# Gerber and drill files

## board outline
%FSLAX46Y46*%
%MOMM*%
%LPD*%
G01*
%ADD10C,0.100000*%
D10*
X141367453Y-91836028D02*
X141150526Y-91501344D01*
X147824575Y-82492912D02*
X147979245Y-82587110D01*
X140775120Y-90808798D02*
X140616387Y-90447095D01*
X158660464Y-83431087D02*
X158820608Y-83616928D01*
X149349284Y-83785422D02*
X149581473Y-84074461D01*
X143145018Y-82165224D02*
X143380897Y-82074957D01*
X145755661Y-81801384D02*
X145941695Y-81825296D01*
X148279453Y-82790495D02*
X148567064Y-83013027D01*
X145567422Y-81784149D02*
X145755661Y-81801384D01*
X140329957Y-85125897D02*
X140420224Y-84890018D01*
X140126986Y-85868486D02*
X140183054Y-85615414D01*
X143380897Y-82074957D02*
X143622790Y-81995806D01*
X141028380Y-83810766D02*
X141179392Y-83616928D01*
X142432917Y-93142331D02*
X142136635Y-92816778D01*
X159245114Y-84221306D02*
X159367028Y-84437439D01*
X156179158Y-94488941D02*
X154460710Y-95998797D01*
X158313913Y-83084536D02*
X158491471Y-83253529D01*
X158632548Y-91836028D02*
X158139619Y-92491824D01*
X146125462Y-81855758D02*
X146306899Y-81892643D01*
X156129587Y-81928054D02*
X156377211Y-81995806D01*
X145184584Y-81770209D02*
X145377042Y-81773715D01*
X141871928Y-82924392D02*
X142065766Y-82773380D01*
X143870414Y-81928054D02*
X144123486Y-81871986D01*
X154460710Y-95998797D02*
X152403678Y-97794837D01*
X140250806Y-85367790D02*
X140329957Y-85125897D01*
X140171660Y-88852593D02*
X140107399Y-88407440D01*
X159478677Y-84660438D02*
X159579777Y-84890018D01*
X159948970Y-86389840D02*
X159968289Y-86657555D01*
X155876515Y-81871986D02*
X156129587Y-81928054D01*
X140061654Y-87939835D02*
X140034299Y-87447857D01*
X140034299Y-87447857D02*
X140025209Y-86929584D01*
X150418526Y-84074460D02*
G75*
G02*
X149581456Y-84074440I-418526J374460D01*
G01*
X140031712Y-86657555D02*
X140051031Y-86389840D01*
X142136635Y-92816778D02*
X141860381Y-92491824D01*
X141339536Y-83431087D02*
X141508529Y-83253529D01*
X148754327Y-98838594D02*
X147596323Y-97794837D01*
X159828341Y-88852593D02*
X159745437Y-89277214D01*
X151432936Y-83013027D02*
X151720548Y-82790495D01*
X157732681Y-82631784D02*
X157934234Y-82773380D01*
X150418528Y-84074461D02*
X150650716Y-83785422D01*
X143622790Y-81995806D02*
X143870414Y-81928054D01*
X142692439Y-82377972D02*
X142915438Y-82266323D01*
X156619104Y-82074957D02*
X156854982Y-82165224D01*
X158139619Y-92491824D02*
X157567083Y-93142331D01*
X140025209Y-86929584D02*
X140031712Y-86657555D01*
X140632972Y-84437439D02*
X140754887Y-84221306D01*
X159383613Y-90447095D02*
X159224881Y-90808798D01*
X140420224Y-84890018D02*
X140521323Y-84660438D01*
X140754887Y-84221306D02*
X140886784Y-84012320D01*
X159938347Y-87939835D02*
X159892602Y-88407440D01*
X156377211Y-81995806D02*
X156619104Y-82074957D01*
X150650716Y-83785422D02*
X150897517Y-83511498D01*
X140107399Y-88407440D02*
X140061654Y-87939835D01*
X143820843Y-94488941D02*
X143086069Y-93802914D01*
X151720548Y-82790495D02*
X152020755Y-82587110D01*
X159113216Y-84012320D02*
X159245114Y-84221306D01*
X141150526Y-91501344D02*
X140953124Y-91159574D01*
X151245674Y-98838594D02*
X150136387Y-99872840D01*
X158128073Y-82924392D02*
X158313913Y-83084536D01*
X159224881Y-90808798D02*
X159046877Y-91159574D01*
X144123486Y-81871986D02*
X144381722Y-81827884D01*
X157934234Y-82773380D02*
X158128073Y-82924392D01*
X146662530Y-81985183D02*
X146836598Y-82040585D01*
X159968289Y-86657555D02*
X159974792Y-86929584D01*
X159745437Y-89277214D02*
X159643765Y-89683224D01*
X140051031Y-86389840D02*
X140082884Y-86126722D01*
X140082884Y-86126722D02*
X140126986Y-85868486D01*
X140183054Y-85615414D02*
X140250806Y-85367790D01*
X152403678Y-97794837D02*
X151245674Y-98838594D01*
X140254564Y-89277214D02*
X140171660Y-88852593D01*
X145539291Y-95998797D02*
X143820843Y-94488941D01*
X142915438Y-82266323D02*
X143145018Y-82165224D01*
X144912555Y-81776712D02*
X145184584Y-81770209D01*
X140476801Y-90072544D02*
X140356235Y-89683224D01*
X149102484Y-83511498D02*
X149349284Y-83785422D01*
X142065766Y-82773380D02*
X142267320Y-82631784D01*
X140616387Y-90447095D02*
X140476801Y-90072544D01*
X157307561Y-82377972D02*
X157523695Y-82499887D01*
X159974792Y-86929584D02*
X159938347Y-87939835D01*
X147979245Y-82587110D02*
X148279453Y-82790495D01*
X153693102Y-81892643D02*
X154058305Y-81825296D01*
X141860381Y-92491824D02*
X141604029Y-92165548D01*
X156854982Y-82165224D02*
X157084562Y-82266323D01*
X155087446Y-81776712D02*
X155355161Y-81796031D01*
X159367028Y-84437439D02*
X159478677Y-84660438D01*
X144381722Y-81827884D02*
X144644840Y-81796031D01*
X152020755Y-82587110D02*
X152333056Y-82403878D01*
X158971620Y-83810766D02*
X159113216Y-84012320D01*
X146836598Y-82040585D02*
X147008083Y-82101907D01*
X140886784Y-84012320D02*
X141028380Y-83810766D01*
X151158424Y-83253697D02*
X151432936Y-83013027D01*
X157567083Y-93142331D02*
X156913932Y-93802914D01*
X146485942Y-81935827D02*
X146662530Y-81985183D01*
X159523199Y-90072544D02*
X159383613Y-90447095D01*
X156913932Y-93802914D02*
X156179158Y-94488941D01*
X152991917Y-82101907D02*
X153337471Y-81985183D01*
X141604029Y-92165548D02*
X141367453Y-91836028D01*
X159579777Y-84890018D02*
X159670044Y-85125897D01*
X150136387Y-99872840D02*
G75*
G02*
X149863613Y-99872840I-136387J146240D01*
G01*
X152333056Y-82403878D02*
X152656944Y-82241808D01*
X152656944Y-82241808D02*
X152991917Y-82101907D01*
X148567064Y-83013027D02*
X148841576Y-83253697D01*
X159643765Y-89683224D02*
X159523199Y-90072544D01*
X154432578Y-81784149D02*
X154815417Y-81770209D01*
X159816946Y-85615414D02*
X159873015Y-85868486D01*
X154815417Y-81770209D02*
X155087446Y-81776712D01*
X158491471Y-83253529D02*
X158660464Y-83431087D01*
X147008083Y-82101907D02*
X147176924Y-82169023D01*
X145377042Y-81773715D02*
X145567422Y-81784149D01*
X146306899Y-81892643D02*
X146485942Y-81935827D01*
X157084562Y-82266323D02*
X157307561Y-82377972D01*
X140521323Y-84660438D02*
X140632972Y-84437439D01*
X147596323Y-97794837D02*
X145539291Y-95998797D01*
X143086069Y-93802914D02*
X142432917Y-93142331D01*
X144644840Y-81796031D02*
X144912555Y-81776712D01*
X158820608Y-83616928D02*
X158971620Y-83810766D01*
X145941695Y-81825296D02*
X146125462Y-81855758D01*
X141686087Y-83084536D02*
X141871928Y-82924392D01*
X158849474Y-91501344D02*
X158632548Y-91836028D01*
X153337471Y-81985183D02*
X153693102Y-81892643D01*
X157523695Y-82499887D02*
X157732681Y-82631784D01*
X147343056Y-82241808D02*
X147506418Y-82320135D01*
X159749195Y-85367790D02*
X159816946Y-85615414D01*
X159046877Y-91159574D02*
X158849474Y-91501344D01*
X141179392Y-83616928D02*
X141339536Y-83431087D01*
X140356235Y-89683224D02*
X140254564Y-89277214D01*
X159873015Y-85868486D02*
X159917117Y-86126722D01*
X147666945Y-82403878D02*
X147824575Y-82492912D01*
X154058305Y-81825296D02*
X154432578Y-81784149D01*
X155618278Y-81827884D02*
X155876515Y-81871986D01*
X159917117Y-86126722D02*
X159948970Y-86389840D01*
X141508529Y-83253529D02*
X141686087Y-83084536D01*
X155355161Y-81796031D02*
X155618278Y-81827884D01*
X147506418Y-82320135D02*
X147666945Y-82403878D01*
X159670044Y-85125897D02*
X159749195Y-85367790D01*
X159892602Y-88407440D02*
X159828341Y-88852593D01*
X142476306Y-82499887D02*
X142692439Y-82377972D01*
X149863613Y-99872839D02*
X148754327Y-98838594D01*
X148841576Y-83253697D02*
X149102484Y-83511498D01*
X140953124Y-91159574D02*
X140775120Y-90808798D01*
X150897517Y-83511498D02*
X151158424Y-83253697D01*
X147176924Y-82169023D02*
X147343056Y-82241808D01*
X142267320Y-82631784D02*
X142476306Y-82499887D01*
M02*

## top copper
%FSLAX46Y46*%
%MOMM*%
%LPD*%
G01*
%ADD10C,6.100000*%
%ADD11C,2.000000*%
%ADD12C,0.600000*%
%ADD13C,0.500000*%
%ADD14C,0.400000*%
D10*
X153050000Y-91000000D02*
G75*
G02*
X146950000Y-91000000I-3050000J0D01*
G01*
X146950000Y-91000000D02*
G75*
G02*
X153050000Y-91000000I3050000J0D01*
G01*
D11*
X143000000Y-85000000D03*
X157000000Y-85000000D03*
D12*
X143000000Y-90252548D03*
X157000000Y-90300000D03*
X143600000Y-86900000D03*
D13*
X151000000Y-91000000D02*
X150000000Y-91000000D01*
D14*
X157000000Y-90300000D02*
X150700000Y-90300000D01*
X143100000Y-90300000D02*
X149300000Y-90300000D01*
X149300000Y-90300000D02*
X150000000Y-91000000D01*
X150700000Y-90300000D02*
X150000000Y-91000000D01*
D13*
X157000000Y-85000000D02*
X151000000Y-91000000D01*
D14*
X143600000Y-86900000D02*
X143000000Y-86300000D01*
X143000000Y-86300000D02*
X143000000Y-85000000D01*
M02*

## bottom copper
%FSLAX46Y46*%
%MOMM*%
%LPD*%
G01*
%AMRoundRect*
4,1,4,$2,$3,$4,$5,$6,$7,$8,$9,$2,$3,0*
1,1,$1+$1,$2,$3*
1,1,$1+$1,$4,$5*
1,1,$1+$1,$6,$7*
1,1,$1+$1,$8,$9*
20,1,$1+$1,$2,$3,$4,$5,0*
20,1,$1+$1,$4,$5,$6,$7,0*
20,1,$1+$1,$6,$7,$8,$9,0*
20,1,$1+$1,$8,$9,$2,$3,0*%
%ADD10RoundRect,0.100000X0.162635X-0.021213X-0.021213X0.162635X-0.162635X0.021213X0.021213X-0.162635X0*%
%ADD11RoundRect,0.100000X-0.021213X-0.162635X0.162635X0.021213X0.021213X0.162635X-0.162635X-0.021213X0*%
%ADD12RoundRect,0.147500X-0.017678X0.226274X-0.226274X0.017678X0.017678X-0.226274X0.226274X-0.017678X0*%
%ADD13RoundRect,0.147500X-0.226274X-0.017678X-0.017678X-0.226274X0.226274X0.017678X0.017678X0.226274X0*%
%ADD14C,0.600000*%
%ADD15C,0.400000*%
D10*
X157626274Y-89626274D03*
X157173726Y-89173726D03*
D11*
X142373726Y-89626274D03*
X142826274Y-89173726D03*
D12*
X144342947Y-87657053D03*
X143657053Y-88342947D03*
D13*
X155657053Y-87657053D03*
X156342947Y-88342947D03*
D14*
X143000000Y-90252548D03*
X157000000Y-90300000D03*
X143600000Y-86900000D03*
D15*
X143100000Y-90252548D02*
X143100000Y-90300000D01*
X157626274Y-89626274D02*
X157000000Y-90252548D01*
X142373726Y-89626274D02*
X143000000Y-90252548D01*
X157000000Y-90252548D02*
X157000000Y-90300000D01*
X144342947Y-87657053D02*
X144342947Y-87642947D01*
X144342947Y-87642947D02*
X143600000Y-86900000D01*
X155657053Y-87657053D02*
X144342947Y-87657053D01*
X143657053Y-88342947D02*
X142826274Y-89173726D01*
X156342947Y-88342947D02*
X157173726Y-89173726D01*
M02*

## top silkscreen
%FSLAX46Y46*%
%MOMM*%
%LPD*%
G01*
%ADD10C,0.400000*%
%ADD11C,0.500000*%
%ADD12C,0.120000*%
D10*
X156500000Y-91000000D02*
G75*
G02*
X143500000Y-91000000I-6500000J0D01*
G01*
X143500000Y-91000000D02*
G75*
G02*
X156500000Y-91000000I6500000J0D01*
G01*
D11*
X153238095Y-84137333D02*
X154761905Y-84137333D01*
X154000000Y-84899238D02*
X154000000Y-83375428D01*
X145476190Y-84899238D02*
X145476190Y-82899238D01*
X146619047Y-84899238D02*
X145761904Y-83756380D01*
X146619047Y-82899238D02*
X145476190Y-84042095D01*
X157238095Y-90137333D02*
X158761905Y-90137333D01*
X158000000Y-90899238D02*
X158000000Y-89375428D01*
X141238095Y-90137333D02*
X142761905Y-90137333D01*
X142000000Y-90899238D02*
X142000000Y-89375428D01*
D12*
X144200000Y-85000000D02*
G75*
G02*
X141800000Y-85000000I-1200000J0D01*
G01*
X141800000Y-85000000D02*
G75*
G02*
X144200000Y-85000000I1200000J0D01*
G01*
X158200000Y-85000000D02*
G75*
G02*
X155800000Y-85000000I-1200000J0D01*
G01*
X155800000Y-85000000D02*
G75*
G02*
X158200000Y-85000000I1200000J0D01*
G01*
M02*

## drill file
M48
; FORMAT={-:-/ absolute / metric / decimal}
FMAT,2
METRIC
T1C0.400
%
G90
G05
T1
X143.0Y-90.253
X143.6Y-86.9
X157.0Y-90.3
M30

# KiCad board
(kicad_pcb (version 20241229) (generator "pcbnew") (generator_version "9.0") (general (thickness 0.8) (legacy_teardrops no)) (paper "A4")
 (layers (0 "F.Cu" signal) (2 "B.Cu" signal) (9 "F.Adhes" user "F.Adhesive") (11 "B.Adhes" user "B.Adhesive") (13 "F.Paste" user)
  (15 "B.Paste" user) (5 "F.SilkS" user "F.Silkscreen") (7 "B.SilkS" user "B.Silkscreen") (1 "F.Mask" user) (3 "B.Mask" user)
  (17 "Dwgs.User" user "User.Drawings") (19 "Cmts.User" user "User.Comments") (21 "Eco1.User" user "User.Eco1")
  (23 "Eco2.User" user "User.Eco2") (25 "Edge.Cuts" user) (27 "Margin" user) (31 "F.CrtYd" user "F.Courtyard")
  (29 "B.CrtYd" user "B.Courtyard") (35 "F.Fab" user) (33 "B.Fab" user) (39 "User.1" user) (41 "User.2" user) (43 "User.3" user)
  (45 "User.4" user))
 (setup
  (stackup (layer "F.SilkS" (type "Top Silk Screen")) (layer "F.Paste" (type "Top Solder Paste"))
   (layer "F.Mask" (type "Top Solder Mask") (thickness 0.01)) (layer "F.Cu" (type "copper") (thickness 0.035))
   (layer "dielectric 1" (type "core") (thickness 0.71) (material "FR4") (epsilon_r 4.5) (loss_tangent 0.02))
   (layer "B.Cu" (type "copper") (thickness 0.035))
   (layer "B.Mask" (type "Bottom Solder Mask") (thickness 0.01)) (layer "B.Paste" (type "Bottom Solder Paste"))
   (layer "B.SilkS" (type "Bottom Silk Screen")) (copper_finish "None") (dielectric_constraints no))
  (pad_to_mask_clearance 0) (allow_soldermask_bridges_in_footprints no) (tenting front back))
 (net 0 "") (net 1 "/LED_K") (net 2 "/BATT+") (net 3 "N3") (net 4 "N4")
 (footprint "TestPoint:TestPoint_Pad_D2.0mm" (layer "F.Cu") (at 143 85)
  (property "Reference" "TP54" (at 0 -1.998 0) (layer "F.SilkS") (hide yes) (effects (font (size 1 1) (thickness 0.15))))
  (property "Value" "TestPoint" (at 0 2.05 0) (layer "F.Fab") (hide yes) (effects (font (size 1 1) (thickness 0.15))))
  (fp_circle (center 0 0) (end 0 1.2) (stroke (width 0.12) (type solid)) (fill no) (layer "F.SilkS"))
  (pad "1" smd circle (at 0 0) (size 2 2) (layers "F.Cu" "F.Mask") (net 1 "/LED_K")))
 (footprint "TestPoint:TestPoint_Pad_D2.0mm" (layer "F.Cu") (at 157 85)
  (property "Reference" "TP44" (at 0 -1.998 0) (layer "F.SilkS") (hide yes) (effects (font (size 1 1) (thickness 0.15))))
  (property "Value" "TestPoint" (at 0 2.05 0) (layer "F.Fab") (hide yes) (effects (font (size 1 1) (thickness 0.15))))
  (fp_circle (center 0 0) (end 0 1.2) (stroke (width 0.12) (type solid)) (fill no) (layer "F.SilkS"))
  (pad "1" smd circle (at 0 0) (size 2 2) (layers "F.Cu" "F.Mask") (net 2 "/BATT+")))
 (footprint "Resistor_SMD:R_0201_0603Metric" (layer "B.Cu") (at 157.4 89.4 135)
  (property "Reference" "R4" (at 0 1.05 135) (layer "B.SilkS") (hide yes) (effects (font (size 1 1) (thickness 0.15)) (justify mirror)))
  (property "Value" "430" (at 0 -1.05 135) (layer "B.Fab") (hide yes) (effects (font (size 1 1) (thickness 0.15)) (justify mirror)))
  (pad "" smd roundrect (at -0.345 0 135) (size 0.318 0.36) (layers "B.Paste") (roundrect_rratio 0.25))
  (pad "" smd roundrect (at 0.345 0 135) (size 0.318 0.36) (layers "B.Paste") (roundrect_rratio 0.25))
  (pad "1" smd roundrect (at -0.32 0 135) (size 0.46 0.4) (layers "B.Cu" "B.Mask") (roundrect_rratio 0.25) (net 2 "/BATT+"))
  (pad "2" smd roundrect (at 0.32 0 135) (size 0.46 0.4) (layers "B.Cu" "B.Mask") (roundrect_rratio 0.25) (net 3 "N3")))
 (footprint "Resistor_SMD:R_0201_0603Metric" (layer "B.Cu") (at 142.6 89.4 45)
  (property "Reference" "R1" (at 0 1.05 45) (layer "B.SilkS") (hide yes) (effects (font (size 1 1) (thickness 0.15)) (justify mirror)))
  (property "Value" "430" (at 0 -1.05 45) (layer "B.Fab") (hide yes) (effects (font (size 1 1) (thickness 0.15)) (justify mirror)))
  (pad "" smd roundrect (at -0.345 0 45) (size 0.318 0.36) (layers "B.Paste") (roundrect_rratio 0.25))
  (pad "" smd roundrect (at 0.345 0 45) (size 0.318 0.36) (layers "B.Paste") (roundrect_rratio 0.25))
  (pad "1" smd roundrect (at -0.32 0 45) (size 0.46 0.4) (layers "B.Cu" "B.Mask") (roundrect_rratio 0.25) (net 2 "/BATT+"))
  (pad "2" smd roundrect (at 0.32 0 45) (size 0.46 0.4) (layers "B.Cu" "B.Mask") (roundrect_rratio 0.25) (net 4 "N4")))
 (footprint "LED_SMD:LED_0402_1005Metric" (layer "B.Cu") (at 144 88 -135)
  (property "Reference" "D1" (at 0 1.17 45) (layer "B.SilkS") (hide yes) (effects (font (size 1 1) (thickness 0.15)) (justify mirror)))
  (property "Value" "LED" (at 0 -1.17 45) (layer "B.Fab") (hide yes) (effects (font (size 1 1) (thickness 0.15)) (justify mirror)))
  (pad "1" smd roundrect (at -0.485 0 225) (size 0.59 0.64) (layers "B.Cu" "B.Mask" "B.Paste") (roundrect_rratio 0.25) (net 1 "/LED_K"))
  (pad "2" smd roundrect (at 0.485 0 225) (size 0.59 0.64) (layers "B.Cu" "B.Mask" "B.Paste") (roundrect_rratio 0.25) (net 4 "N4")))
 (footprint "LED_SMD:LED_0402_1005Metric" (layer "B.Cu") (at 156 88 -45)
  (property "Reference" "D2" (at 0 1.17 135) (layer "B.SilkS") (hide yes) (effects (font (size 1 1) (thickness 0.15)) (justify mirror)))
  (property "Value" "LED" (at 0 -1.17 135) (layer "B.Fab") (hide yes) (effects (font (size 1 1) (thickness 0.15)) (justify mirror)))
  (pad "1" smd roundrect (at -0.485 0 315) (size 0.59 0.64) (layers "B.Cu" "B.Mask" "B.Paste") (roundrect_rratio 0.25) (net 1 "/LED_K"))
  (pad "2" smd roundrect (at 0.485 0 315) (size 0.59 0.64) (layers "B.Cu" "B.Mask" "B.Paste") (roundrect_rratio 0.25) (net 3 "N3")))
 (gr_circle (center 150 91) (end 156 91) (stroke (width 0.2) (type solid)) (fill yes) (layers "F.Cu" "F.Mask") (net 2))
 (gr_circle (center 150 91) (end 143.5 91) (stroke (width 0.4) (type solid)) (fill no) (layer "F.SilkS"))
 (gr_line (start 141.367453 91.836028) (end 141.150526 91.501344) (stroke (width 0.1) (type default)) (layer "Edge.Cuts"))
 (gr_line (start 147.824575 82.492912) (end 147.979245 82.58711) (stroke (width 0.1) (type default)) (layer "Edge.Cuts"))
 (gr_line (start 140.77512 90.808798) (end 140.616387 90.447095) (stroke (width 0.1) (type default)) (layer "Edge.Cuts"))
 (gr_line (start 158.660464 83.431087) (end 158.820608 83.616928) (stroke (width 0.1) (type default)) (layer "Edge.Cuts"))
 (gr_line (start 149.349284 83.785422) (end 149.581473 84.074461) (stroke (width 0.1) (type default)) (layer "Edge.Cuts"))
 (gr_line (start 143.145018 82.165224) (end 143.380897 82.074957) (stroke (width 0.1) (type default)) (layer "Edge.Cuts"))
 (gr_line (start 145.755661 81.801384) (end 145.941695 81.825296) (stroke (width 0.1) (type default)) (layer "Edge.Cuts"))
 (gr_line (start 148.279453 82.790495) (end 148.567064 83.013027) (stroke (width 0.1) (type default)) (layer "Edge.Cuts"))
 (gr_line (start 145.567422 81.784149) (end 145.755661 81.801384) (stroke (width 0.1) (type default)) (layer "Edge.Cuts"))
 (gr_line (start 140.329957 85.125897) (end 140.420224 84.890018) (stroke (width 0.1) (type default)) (layer "Edge.Cuts"))
 (gr_line (start 140.126986 85.868486) (end 140.183054 85.615414) (stroke (width 0.1) (type default)) (layer "Edge.Cuts"))
 (gr_line (start 143.380897 82.074957) (end 143.62279 81.995806) (stroke (width 0.1) (type default)) (layer "Edge.Cuts"))
 (gr_line (start 141.02838 83.810766) (end 141.179392 83.616928) (stroke (width 0.1) (type default)) (layer "Edge.Cuts"))
 (gr_line (start 142.432917 93.142331) (end 142.136635 92.816778) (stroke (width 0.1) (type default)) (layer "Edge.Cuts"))
 (gr_line (start 159.245114 84.221306) (end 159.367028 84.437439) (stroke (width 0.1) (type default)) (layer "Edge.Cuts"))
 (gr_line (start 156.179158 94.488941) (end 154.46071 95.998797) (stroke (width 0.1) (type default)) (layer "Edge.Cuts"))
 (gr_line (start 158.313913 83.084536) (end 158.491471 83.253529) (stroke (width 0.1) (type default)) (layer "Edge.Cuts"))
 (gr_line (start 158.632548 91.836028) (end 158.139619 92.491824) (stroke (width 0.1) (type default)) (layer "Edge.Cuts"))
 (gr_line (start 146.125462 81.855758) (end 146.306899 81.892643) (stroke (width 0.1) (type default)) (layer "Edge.Cuts"))
 (gr_line (start 156.129587 81.928054) (end 156.377211 81.995806) (stroke (width 0.1) (type default)) (layer "Edge.Cuts"))
 (gr_line (start 145.184584 81.770209) (end 145.377042 81.773715) (stroke (width 0.1) (type default)) (layer "Edge.Cuts"))
 (gr_line (start 141.871928 82.924392) (end 142.065766 82.77338) (stroke (width 0.1) (type default)) (layer "Edge.Cuts"))
 (gr_line (start 143.870414 81.928054) (end 144.123486 81.871986) (stroke (width 0.1) (type default)) (layer "Edge.Cuts"))
 (gr_line (start 154.46071 95.998797) (end 152.403678 97.794837) (stroke (width 0.1) (type default)) (layer "Edge.Cuts"))
 (gr_line (start 140.250806 85.36779) (end 140.329957 85.125897) (stroke (width 0.1) (type default)) (layer "Edge.Cuts"))
 (gr_line (start 140.17166 88.852593) (end 140.107399 88.40744) (stroke (width 0.1) (type default)) (layer "Edge.Cuts"))
 (gr_line (start 159.478677 84.660438) (end 159.579777 84.890018) (stroke (width 0.1) (type default)) (layer "Edge.Cuts"))
 (gr_line (start 159.94897 86.38984) (end 159.968289 86.657555) (stroke (width 0.1) (type default)) (layer "Edge.Cuts"))
 (gr_line (start 155.876515 81.871986) (end 156.129587 81.928054) (stroke (width 0.1) (type default)) (layer "Edge.Cuts"))
 (gr_line (start 140.061654 87.939835) (end 140.034299 87.447857) (stroke (width 0.1) (type default)) (layer "Edge.Cuts"))
 (gr_line (start 140.034299 87.447857) (end 140.025209 86.929584) (stroke (width 0.1) (type default)) (layer "Edge.Cuts"))
 (gr_arc (start 150.418526 84.07446) (mid 149.999986 84.261587) (end 149.581456 84.07444) (stroke (width 0.1) (type solid))
  (layer "Edge.Cuts"))
 (gr_line (start 140.031712 86.657555) (end 140.051031 86.38984) (stroke (width 0.1) (type default)) (layer "Edge.Cuts"))
 (gr_line (start 142.136635 92.816778) (end 141.860381 92.491824) (stroke (width 0.1) (type default)) (layer "Edge.Cuts"))
 (gr_line (start 141.339536 83.431087) (end 141.508529 83.253529) (stroke (width 0.1) (type default)) (layer "Edge.Cuts"))
 (gr_line (start 148.754327 98.838594) (end 147.596323 97.794837) (stroke (width 0.1) (type default)) (layer "Edge.Cuts"))
 (gr_line (start 159.828341 88.852593) (end 159.745437 89.277214) (stroke (width 0.1) (type default)) (layer "Edge.Cuts"))
 (gr_line (start 151.432936 83.013027) (end 151.720548 82.790495) (stroke (width 0.1) (type default)) (layer "Edge.Cuts"))
 (gr_line (start 157.732681 82.631784) (end 157.934234 82.77338) (stroke (width 0.1) (type default)) (layer "Edge.Cuts"))
 (gr_line (start 150.418528 84.074461) (end 150.650716 83.785422) (stroke (width 0.1) (type default)) (layer "Edge.Cuts"))
 (gr_line (start 143.62279 81.995806) (end 143.870414 81.928054) (stroke (width 0.1) (type default)) (layer "Edge.Cuts"))
 (gr_line (start 142.692439 82.377972) (end 142.915438 82.266323) (stroke (width 0.1) (type default)) (layer "Edge.Cuts"))
 (gr_line (start 156.619104 82.074957) (end 156.854982 82.165224) (stroke (width 0.1) (type default)) (layer "Edge.Cuts"))
 (gr_line (start 158.139619 92.491824) (end 157.567083 93.142331) (stroke (width 0.1) (type default)) (layer "Edge.Cuts"))
 (gr_line (start 140.025209 86.929584) (end 140.031712 86.657555) (stroke (width 0.1) (type default)) (layer "Edge.Cuts"))
 (gr_line (start 140.632972 84.437439) (end 140.754887 84.221306) (stroke (width 0.1) (type default)) (layer "Edge.Cuts"))
 (gr_line (start 159.383613 90.447095) (end 159.224881 90.808798) (stroke (width 0.1) (type default)) (layer "Edge.Cuts"))
 (gr_line (start 140.420224 84.890018) (end 140.521323 84.660438) (stroke (width 0.1) (type default)) (layer "Edge.Cuts"))
 (gr_line (start 140.754887 84.221306) (end 140.886784 84.01232) (stroke (width 0.1) (type default)) (layer "Edge.Cuts"))
 (gr_line (start 159.938347 87.939835) (end 159.892602 88.40744) (stroke (width 0.1) (type default)) (layer "Edge.Cuts"))
 (gr_line (start 156.377211 81.995806) (end 156.619104 82.074957) (stroke (width 0.1) (type default)) (layer "Edge.Cuts"))
 (gr_line (start 150.650716 83.785422) (end 150.897517 83.511498) (stroke (width 0.1) (type default)) (layer "Edge.Cuts"))
 (gr_line (start 140.107399 88.40744) (end 140.061654 87.939835) (stroke (width 0.1) (type default)) (layer "Edge.Cuts"))
 (gr_line (start 143.820843 94.488941) (end 143.086069 93.802914) (stroke (width 0.1) (type default)) (layer "Edge.Cuts"))
 (gr_line (start 151.720548 82.790495) (end 152.020755 82.58711) (stroke (width 0.1) (type default)) (layer "Edge.Cuts"))
 (gr_line (start 159.113216 84.01232) (end 159.245114 84.221306) (stroke (width 0.1) (type default)) (layer "Edge.Cuts"))
 (gr_line (start 141.150526 91.501344) (end 140.953124 91.159574) (stroke (width 0.1) (type default)) (layer "Edge.Cuts"))
 (gr_line (start 151.245674 98.838594) (end 150.136387 99.87284) (stroke (width 0.1) (type default)) (layer "Edge.Cuts"))
 (gr_line (start 158.128073 82.924392) (end 158.313913 83.084536) (stroke (width 0.1) (type default)) (layer "Edge.Cuts"))
 (gr_line (start 159.224881 90.808798) (end 159.046877 91.159574) (stroke (width 0.1) (type default)) (layer "Edge.Cuts"))
 (gr_line (start 144.123486 81.871986) (end 144.381722 81.827884) (stroke (width 0.1) (type default)) (layer "Edge.Cuts"))
 (gr_line (start 157.934234 82.77338) (end 158.128073 82.924392) (stroke (width 0.1) (type default)) (layer "Edge.Cuts"))
 (gr_line (start 146.66253 81.985183) (end 146.836598 82.040585) (stroke (width 0.1) (type default)) (layer "Edge.Cuts"))
 (gr_line (start 159.968289 86.657555) (end 159.974792 86.929584) (stroke (width 0.1) (type default)) (layer "Edge.Cuts"))
 (gr_line (start 159.745437 89.277214) (end 159.643765 89.683224) (stroke (width 0.1) (type default)) (layer "Edge.Cuts"))
 (gr_line (start 140.051031 86.38984) (end 140.082884 86.126722) (stroke (width 0.1) (type default)) (layer "Edge.Cuts"))
 (gr_line (start 140.082884 86.126722) (end 140.126986 85.868486) (stroke (width 0.1) (type default)) (layer "Edge.Cuts"))
 (gr_line (start 140.183054 85.615414) (end 140.250806 85.36779) (stroke (width 0.1) (type default)) (layer "Edge.Cuts"))
 (gr_line (start 152.403678 97.794837) (end 151.245674 98.838594) (stroke (width 0.1) (type default)) (layer "Edge.Cuts"))
 (gr_line (start 140.254564 89.277214) (end 140.17166 88.852593) (stroke (width 0.1) (type default)) (layer "Edge.Cuts"))
 (gr_line (start 145.539291 95.998797) (end 143.820843 94.488941) (stroke (width 0.1) (type default)) (layer "Edge.Cuts"))
 (gr_line (start 142.915438 82.266323) (end 143.145018 82.165224) (stroke (width 0.1) (type default)) (layer "Edge.Cuts"))
 (gr_line (start 144.912555 81.776712) (end 145.184584 81.770209) (stroke (width 0.1) (type default)) (layer "Edge.Cuts"))
 (gr_line (start 140.476801 90.072544) (end 140.356235 89.683224) (stroke (width 0.1) (type default)) (layer "Edge.Cuts"))
 (gr_line (start 149.102484 83.511498) (end 149.349284 83.785422) (stroke (width 0.1) (type default)) (layer "Edge.Cuts"))
 (gr_line (start 142.065766 82.77338) (end 142.26732 82.631784) (stroke (width 0.1) (type default)) (layer "Edge.Cuts"))
 (gr_line (start 140.616387 90.447095) (end 140.476801 90.072544) (stroke (width 0.1) (type default)) (layer "Edge.Cuts"))
 (gr_line (start 157.307561 82.377972) (end 157.523695 82.499887) (stroke (width 0.1) (type default)) (layer "Edge.Cuts"))
 (gr_line (start 159.974792 86.929584) (end 159.938347 87.939835) (stroke (width 0.1) (type default)) (layer "Edge.Cuts"))
 (gr_line (start 147.979245 82.58711) (end 148.279453 82.790495) (stroke (width 0.1) (type default)) (layer "Edge.Cuts"))
 (gr_line (start 153.693102 81.892643) (end 154.058305 81.825296) (stroke (width 0.1) (type default)) (layer "Edge.Cuts"))
 (gr_line (start 141.860381 92.491824) (end 141.604029 92.165548) (stroke (width 0.1) (type default)) (layer "Edge.Cuts"))
 (gr_line (start 156.854982 82.165224) (end 157.084562 82.266323) (stroke (width 0.1) (type default)) (layer "Edge.Cuts"))
 (gr_line (start 155.087446 81.776712) (end 155.355161 81.796031) (stroke (width 0.1) (type default)) (layer "Edge.Cuts"))
 (gr_line (start 159.367028 84.437439) (end 159.478677 84.660438) (stroke (width 0.1) (type default)) (layer "Edge.Cuts"))
 (gr_line (start 144.381722 81.827884) (end 144.64484 81.796031) (stroke (width 0.1) (type default)) (layer "Edge.Cuts"))
 (gr_line (start 152.020755 82.58711) (end 152.333056 82.403878) (stroke (width 0.1) (type default)) (layer "Edge.Cuts"))
 (gr_line (start 158.97162 83.810766) (end 159.113216 84.01232) (stroke (width 0.1) (type default)) (layer "Edge.Cuts"))
 (gr_line (start 146.836598 82.040585) (end 147.008083 82.101907) (stroke (width 0.1) (type default)) (layer "Edge.Cuts"))
 (gr_line (start 140.886784 84.01232) (end 141.02838 83.810766) (stroke (width 0.1) (type default)) (layer "Edge.Cuts"))
 (gr_line (start 151.158424 83.253697) (end 151.432936 83.013027) (stroke (width 0.1) (type default)) (layer "Edge.Cuts"))
 (gr_line (start 157.567083 93.142331) (end 156.913932 93.802914) (stroke (width 0.1) (type default)) (layer "Edge.Cuts"))
 (gr_line (start 146.485942 81.935827) (end 146.66253 81.985183) (stroke (width 0.1) (type default)) (layer "Edge.Cuts"))
 (gr_line (start 159.523199 90.072544) (end 159.383613 90.447095) (stroke (width 0.1) (type default)) (layer "Edge.Cuts"))
 (gr_line (start 156.913932 93.802914) (end 156.179158 94.488941) (stroke (width 0.1) (type default)) (layer "Edge.Cuts"))
 (gr_line (start 152.991917 82.101907) (end 153.337471 81.985183) (stroke (width 0.1) (type default)) (layer "Edge.Cuts"))
 (gr_line (start 141.604029 92.165548) (end 141.367453 91.836028) (stroke (width 0.1) (type default)) (layer "Edge.Cuts"))
 (gr_line (start 159.579777 84.890018) (end 159.670044 85.125897) (stroke (width 0.1) (type default)) (layer "Edge.Cuts"))
 (gr_arc (start 150.136387 99.87284) (mid 150 99.926569) (end 149.863613 99.872839) (stroke (width 0.1) (type default)) (layer "Edge.Cuts"))
 (gr_line (start 152.333056 82.403878) (end 152.656944 82.241808) (stroke (width 0.1) (type default)) (layer "Edge.Cuts"))
 (gr_line (start 152.656944 82.241808) (end 152.991917 82.101907) (stroke (width 0.1) (type default)) (layer "Edge.Cuts"))
 (gr_line (start 148.567064 83.013027) (end 148.841576 83.253697) (stroke (width 0.1) (type default)) (layer "Edge.Cuts"))
 (gr_line (start 159.643765 89.683224) (end 159.523199 90.072544) (stroke (width 0.1) (type default)) (layer "Edge.Cuts"))
 (gr_line (start 154.432578 81.784149) (end 154.815417 81.770209) (stroke (width 0.1) (type default)) (layer "Edge.Cuts"))
 (gr_line (start 159.816946 85.615414) (end 159.873015 85.868486) (stroke (width 0.1) (type default)) (layer "Edge.Cuts"))
 (gr_line (start 154.815417 81.770209) (end 155.087446 81.776712) (stroke (width 0.1) (type default)) (layer "Edge.Cuts"))
 (gr_line (start 158.491471 83.253529) (end 158.660464 83.431087) (stroke (width 0.1) (type default)) (layer "Edge.Cuts"))
 (gr_line (start 147.008083 82.101907) (end 147.176924 82.169023) (stroke (width 0.1) (type default)) (layer "Edge.Cuts"))
 (gr_line (start 145.377042 81.773715) (end 145.567422 81.784149) (stroke (width 0.1) (type default)) (layer "Edge.Cuts"))
 (gr_line (start 146.306899 81.892643) (end 146.485942 81.935827) (stroke (width 0.1) (type default)) (layer "Edge.Cuts"))
 (gr_line (start 157.084562 82.266323) (end 157.307561 82.377972) (stroke (width 0.1) (type default)) (layer "Edge.Cuts"))
 (gr_line (start 140.521323 84.660438) (end 140.632972 84.437439) (stroke (width 0.1) (type default)) (layer "Edge.Cuts"))
 (gr_line (start 147.596323 97.794837) (end 145.539291 95.998797) (stroke (width 0.1) (type default)) (layer "Edge.Cuts"))
 (gr_line (start 143.086069 93.802914) (end 142.432917 93.142331) (stroke (width 0.1) (type default)) (layer "Edge.Cuts"))
 (gr_line (start 144.64484 81.796031) (end 144.912555 81.776712) (stroke (width 0.1) (type default)) (layer "Edge.Cuts"))
 (gr_line (start 158.820608 83.616928) (end 158.97162 83.810766) (stroke (width 0.1) (type default)) (layer "Edge.Cuts"))
 (gr_line (start 145.941695 81.825296) (end 146.125462 81.855758) (stroke (width 0.1) (type default)) (layer "Edge.Cuts"))
 (gr_line (start 141.686087 83.084536) (end 141.871928 82.924392) (stroke (width 0.1) (type default)) (layer "Edge.Cuts"))
 (gr_line (start 158.849474 91.501344) (end 158.632548 91.836028) (stroke (width 0.1) (type default)) (layer "Edge.Cuts"))
 (gr_line (start 153.337471 81.985183) (end 153.693102 81.892643) (stroke (width 0.1) (type default)) (layer "Edge.Cuts"))
 (gr_line (start 157.523695 82.499887) (end 157.732681 82.631784) (stroke (width 0.1) (type default)) (layer "Edge.Cuts"))
 (gr_line (start 147.343056 82.241808) (end 147.506418 82.320135) (stroke (width 0.1) (type default)) (layer "Edge.Cuts"))
 (gr_line (start 159.749195 85.36779) (end 159.816946 85.615414) (stroke (width 0.1) (type default)) (layer "Edge.Cuts"))
 (gr_line (start 159.046877 91.159574) (end 158.849474 91.501344) (stroke (width 0.1) (type default)) (layer "Edge.Cuts"))
 (gr_line (start 141.179392 83.616928) (end 141.339536 83.431087) (stroke (width 0.1) (type default)) (layer "Edge.Cuts"))
 (gr_line (start 140.356235 89.683224) (end 140.254564 89.277214) (stroke (width 0.1) (type default)) (layer "Edge.Cuts"))
 (gr_line (start 159.873015 85.868486) (end 159.917117 86.126722) (stroke (width 0.1) (type default)) (layer "Edge.Cuts"))
 (gr_line (start 147.666945 82.403878) (end 147.824575 82.492912) (stroke (width 0.1) (type default)) (layer "Edge.Cuts"))
 (gr_line (start 154.058305 81.825296) (end 154.432578 81.784149) (stroke (width 0.1) (type default)) (layer "Edge.Cuts"))
 (gr_line (start 155.618278 81.827884) (end 155.876515 81.871986) (stroke (width 0.1) (type default)) (layer "Edge.Cuts"))
 (gr_line (start 159.917117 86.126722) (end 159.94897 86.38984) (stroke (width 0.1) (type default)) (layer "Edge.Cuts"))
 (gr_line (start 141.508529 83.253529) (end 141.686087 83.084536) (stroke (width 0.1) (type default)) (layer "Edge.Cuts"))
 (gr_line (start 155.355161 81.796031) (end 155.618278 81.827884) (stroke (width 0.1) (type default)) (layer "Edge.Cuts"))
 (gr_line (start 147.506418 82.320135) (end 147.666945 82.403878) (stroke (width 0.1) (type default)) (layer "Edge.Cuts"))
 (gr_line (start 159.670044 85.125897) (end 159.749195 85.36779) (stroke (width 0.1) (type default)) (layer "Edge.Cuts"))
 (gr_line (start 159.892602 88.40744) (end 159.828341 88.852593) (stroke (width 0.1) (type default)) (layer "Edge.Cuts"))
 (gr_line (start 142.476306 82.499887) (end 142.692439 82.377972) (stroke (width 0.1) (type default)) (layer "Edge.Cuts"))
 (gr_line (start 149.863613 99.872839) (end 148.754327 98.838594) (stroke (width 0.1) (type default)) (layer "Edge.Cuts"))
 (gr_line (start 148.841576 83.253697) (end 149.102484 83.511498) (stroke (width 0.1) (type default)) (layer "Edge.Cuts"))
 (gr_line (start 140.953124 91.159574) (end 140.77512 90.808798) (stroke (width 0.1) (type default)) (layer "Edge.Cuts"))
 (gr_line (start 150.897517 83.511498) (end 151.158424 83.253697) (stroke (width 0.1) (type default)) (layer "Edge.Cuts"))
 (gr_line (start 147.176924 82.169023) (end 147.343056 82.241808) (stroke (width 0.1) (type default)) (layer "Edge.Cuts"))
 (gr_line (start 142.26732 82.631784) (end 142.476306 82.499887) (stroke (width 0.1) (type default)) (layer "Edge.Cuts"))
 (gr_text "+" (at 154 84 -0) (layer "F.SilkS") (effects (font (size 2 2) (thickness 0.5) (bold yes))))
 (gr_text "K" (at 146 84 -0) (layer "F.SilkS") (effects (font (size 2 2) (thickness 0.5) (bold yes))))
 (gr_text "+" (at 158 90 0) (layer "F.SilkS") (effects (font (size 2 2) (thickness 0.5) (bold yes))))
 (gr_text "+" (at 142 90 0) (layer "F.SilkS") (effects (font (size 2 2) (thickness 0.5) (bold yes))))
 (segment (start 151 91) (end 150 91) (width 0.5) (layer "F.Cu") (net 2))
 (segment (start 157 90.3) (end 150.7 90.3) (width 0.4) (layer "F.Cu") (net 2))
 (segment (start 143.1 90.3) (end 149.3 90.3) (width 0.4) (layer "F.Cu") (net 2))
 (segment (start 149.3 90.3) (end 150 91) (width 0.4) (layer "F.Cu") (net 2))
 (segment (start 150.7 90.3) (end 150 91) (width 0.4) (layer "F.Cu") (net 2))
 (segment (start 157 85) (end 151 91) (width 0.5) (layer "F.Cu") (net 2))
 (via (at 143 90.252548) (size 0.6) (drill 0.4) (layers "F.Cu" "B.Cu") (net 2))
 (via (at 157 90.3) (size 0.6) (drill 0.4) (layers "F.Cu" "B.Cu") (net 2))
 (segment (start 143.1 90.252548) (end 143.1 90.3) (width 0.4) (layer "B.Cu") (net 2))
 (segment (start 157.626274 89.626274) (end 157 90.252548) (width 0.4) (layer "B.Cu") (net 2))
 (segment (start 142.373726 89.626274) (end 143 90.252548) (width 0.4) (layer "B.Cu") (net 2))
 (segment (start 157 90.252548) (end 157 90.3) (width 0.4) (layer "B.Cu") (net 2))
 (segment (start 143.6 86.9) (end 143 86.3) (width 0.4) (layer "F.Cu") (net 1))
 (segment (start 143 86.3) (end 143 85) (width 0.4) (layer "F.Cu") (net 1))
 (via (at 143.6 86.9) (size 0.6) (drill 0.4) (layers "F.Cu" "B.Cu") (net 1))
 (segment (start 144.342947 87.657053) (end 144.342947 87.642947) (width 0.4) (layer "B.Cu") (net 1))
 (segment (start 144.342947 87.642947) (end 143.6 86.9) (width 0.4) (layer "B.Cu") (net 1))
 (segment (start 155.657053 87.657053) (end 144.342947 87.657053) (width 0.4) (layer "B.Cu") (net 1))
 (segment (start 143.657053 88.342947) (end 142.826274 89.173726) (width 0.4) (layer "B.Cu") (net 4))
 (segment (start 156.342947 88.342947) (end 157.173726 89.173726) (width 0.4) (layer "B.Cu") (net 3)))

